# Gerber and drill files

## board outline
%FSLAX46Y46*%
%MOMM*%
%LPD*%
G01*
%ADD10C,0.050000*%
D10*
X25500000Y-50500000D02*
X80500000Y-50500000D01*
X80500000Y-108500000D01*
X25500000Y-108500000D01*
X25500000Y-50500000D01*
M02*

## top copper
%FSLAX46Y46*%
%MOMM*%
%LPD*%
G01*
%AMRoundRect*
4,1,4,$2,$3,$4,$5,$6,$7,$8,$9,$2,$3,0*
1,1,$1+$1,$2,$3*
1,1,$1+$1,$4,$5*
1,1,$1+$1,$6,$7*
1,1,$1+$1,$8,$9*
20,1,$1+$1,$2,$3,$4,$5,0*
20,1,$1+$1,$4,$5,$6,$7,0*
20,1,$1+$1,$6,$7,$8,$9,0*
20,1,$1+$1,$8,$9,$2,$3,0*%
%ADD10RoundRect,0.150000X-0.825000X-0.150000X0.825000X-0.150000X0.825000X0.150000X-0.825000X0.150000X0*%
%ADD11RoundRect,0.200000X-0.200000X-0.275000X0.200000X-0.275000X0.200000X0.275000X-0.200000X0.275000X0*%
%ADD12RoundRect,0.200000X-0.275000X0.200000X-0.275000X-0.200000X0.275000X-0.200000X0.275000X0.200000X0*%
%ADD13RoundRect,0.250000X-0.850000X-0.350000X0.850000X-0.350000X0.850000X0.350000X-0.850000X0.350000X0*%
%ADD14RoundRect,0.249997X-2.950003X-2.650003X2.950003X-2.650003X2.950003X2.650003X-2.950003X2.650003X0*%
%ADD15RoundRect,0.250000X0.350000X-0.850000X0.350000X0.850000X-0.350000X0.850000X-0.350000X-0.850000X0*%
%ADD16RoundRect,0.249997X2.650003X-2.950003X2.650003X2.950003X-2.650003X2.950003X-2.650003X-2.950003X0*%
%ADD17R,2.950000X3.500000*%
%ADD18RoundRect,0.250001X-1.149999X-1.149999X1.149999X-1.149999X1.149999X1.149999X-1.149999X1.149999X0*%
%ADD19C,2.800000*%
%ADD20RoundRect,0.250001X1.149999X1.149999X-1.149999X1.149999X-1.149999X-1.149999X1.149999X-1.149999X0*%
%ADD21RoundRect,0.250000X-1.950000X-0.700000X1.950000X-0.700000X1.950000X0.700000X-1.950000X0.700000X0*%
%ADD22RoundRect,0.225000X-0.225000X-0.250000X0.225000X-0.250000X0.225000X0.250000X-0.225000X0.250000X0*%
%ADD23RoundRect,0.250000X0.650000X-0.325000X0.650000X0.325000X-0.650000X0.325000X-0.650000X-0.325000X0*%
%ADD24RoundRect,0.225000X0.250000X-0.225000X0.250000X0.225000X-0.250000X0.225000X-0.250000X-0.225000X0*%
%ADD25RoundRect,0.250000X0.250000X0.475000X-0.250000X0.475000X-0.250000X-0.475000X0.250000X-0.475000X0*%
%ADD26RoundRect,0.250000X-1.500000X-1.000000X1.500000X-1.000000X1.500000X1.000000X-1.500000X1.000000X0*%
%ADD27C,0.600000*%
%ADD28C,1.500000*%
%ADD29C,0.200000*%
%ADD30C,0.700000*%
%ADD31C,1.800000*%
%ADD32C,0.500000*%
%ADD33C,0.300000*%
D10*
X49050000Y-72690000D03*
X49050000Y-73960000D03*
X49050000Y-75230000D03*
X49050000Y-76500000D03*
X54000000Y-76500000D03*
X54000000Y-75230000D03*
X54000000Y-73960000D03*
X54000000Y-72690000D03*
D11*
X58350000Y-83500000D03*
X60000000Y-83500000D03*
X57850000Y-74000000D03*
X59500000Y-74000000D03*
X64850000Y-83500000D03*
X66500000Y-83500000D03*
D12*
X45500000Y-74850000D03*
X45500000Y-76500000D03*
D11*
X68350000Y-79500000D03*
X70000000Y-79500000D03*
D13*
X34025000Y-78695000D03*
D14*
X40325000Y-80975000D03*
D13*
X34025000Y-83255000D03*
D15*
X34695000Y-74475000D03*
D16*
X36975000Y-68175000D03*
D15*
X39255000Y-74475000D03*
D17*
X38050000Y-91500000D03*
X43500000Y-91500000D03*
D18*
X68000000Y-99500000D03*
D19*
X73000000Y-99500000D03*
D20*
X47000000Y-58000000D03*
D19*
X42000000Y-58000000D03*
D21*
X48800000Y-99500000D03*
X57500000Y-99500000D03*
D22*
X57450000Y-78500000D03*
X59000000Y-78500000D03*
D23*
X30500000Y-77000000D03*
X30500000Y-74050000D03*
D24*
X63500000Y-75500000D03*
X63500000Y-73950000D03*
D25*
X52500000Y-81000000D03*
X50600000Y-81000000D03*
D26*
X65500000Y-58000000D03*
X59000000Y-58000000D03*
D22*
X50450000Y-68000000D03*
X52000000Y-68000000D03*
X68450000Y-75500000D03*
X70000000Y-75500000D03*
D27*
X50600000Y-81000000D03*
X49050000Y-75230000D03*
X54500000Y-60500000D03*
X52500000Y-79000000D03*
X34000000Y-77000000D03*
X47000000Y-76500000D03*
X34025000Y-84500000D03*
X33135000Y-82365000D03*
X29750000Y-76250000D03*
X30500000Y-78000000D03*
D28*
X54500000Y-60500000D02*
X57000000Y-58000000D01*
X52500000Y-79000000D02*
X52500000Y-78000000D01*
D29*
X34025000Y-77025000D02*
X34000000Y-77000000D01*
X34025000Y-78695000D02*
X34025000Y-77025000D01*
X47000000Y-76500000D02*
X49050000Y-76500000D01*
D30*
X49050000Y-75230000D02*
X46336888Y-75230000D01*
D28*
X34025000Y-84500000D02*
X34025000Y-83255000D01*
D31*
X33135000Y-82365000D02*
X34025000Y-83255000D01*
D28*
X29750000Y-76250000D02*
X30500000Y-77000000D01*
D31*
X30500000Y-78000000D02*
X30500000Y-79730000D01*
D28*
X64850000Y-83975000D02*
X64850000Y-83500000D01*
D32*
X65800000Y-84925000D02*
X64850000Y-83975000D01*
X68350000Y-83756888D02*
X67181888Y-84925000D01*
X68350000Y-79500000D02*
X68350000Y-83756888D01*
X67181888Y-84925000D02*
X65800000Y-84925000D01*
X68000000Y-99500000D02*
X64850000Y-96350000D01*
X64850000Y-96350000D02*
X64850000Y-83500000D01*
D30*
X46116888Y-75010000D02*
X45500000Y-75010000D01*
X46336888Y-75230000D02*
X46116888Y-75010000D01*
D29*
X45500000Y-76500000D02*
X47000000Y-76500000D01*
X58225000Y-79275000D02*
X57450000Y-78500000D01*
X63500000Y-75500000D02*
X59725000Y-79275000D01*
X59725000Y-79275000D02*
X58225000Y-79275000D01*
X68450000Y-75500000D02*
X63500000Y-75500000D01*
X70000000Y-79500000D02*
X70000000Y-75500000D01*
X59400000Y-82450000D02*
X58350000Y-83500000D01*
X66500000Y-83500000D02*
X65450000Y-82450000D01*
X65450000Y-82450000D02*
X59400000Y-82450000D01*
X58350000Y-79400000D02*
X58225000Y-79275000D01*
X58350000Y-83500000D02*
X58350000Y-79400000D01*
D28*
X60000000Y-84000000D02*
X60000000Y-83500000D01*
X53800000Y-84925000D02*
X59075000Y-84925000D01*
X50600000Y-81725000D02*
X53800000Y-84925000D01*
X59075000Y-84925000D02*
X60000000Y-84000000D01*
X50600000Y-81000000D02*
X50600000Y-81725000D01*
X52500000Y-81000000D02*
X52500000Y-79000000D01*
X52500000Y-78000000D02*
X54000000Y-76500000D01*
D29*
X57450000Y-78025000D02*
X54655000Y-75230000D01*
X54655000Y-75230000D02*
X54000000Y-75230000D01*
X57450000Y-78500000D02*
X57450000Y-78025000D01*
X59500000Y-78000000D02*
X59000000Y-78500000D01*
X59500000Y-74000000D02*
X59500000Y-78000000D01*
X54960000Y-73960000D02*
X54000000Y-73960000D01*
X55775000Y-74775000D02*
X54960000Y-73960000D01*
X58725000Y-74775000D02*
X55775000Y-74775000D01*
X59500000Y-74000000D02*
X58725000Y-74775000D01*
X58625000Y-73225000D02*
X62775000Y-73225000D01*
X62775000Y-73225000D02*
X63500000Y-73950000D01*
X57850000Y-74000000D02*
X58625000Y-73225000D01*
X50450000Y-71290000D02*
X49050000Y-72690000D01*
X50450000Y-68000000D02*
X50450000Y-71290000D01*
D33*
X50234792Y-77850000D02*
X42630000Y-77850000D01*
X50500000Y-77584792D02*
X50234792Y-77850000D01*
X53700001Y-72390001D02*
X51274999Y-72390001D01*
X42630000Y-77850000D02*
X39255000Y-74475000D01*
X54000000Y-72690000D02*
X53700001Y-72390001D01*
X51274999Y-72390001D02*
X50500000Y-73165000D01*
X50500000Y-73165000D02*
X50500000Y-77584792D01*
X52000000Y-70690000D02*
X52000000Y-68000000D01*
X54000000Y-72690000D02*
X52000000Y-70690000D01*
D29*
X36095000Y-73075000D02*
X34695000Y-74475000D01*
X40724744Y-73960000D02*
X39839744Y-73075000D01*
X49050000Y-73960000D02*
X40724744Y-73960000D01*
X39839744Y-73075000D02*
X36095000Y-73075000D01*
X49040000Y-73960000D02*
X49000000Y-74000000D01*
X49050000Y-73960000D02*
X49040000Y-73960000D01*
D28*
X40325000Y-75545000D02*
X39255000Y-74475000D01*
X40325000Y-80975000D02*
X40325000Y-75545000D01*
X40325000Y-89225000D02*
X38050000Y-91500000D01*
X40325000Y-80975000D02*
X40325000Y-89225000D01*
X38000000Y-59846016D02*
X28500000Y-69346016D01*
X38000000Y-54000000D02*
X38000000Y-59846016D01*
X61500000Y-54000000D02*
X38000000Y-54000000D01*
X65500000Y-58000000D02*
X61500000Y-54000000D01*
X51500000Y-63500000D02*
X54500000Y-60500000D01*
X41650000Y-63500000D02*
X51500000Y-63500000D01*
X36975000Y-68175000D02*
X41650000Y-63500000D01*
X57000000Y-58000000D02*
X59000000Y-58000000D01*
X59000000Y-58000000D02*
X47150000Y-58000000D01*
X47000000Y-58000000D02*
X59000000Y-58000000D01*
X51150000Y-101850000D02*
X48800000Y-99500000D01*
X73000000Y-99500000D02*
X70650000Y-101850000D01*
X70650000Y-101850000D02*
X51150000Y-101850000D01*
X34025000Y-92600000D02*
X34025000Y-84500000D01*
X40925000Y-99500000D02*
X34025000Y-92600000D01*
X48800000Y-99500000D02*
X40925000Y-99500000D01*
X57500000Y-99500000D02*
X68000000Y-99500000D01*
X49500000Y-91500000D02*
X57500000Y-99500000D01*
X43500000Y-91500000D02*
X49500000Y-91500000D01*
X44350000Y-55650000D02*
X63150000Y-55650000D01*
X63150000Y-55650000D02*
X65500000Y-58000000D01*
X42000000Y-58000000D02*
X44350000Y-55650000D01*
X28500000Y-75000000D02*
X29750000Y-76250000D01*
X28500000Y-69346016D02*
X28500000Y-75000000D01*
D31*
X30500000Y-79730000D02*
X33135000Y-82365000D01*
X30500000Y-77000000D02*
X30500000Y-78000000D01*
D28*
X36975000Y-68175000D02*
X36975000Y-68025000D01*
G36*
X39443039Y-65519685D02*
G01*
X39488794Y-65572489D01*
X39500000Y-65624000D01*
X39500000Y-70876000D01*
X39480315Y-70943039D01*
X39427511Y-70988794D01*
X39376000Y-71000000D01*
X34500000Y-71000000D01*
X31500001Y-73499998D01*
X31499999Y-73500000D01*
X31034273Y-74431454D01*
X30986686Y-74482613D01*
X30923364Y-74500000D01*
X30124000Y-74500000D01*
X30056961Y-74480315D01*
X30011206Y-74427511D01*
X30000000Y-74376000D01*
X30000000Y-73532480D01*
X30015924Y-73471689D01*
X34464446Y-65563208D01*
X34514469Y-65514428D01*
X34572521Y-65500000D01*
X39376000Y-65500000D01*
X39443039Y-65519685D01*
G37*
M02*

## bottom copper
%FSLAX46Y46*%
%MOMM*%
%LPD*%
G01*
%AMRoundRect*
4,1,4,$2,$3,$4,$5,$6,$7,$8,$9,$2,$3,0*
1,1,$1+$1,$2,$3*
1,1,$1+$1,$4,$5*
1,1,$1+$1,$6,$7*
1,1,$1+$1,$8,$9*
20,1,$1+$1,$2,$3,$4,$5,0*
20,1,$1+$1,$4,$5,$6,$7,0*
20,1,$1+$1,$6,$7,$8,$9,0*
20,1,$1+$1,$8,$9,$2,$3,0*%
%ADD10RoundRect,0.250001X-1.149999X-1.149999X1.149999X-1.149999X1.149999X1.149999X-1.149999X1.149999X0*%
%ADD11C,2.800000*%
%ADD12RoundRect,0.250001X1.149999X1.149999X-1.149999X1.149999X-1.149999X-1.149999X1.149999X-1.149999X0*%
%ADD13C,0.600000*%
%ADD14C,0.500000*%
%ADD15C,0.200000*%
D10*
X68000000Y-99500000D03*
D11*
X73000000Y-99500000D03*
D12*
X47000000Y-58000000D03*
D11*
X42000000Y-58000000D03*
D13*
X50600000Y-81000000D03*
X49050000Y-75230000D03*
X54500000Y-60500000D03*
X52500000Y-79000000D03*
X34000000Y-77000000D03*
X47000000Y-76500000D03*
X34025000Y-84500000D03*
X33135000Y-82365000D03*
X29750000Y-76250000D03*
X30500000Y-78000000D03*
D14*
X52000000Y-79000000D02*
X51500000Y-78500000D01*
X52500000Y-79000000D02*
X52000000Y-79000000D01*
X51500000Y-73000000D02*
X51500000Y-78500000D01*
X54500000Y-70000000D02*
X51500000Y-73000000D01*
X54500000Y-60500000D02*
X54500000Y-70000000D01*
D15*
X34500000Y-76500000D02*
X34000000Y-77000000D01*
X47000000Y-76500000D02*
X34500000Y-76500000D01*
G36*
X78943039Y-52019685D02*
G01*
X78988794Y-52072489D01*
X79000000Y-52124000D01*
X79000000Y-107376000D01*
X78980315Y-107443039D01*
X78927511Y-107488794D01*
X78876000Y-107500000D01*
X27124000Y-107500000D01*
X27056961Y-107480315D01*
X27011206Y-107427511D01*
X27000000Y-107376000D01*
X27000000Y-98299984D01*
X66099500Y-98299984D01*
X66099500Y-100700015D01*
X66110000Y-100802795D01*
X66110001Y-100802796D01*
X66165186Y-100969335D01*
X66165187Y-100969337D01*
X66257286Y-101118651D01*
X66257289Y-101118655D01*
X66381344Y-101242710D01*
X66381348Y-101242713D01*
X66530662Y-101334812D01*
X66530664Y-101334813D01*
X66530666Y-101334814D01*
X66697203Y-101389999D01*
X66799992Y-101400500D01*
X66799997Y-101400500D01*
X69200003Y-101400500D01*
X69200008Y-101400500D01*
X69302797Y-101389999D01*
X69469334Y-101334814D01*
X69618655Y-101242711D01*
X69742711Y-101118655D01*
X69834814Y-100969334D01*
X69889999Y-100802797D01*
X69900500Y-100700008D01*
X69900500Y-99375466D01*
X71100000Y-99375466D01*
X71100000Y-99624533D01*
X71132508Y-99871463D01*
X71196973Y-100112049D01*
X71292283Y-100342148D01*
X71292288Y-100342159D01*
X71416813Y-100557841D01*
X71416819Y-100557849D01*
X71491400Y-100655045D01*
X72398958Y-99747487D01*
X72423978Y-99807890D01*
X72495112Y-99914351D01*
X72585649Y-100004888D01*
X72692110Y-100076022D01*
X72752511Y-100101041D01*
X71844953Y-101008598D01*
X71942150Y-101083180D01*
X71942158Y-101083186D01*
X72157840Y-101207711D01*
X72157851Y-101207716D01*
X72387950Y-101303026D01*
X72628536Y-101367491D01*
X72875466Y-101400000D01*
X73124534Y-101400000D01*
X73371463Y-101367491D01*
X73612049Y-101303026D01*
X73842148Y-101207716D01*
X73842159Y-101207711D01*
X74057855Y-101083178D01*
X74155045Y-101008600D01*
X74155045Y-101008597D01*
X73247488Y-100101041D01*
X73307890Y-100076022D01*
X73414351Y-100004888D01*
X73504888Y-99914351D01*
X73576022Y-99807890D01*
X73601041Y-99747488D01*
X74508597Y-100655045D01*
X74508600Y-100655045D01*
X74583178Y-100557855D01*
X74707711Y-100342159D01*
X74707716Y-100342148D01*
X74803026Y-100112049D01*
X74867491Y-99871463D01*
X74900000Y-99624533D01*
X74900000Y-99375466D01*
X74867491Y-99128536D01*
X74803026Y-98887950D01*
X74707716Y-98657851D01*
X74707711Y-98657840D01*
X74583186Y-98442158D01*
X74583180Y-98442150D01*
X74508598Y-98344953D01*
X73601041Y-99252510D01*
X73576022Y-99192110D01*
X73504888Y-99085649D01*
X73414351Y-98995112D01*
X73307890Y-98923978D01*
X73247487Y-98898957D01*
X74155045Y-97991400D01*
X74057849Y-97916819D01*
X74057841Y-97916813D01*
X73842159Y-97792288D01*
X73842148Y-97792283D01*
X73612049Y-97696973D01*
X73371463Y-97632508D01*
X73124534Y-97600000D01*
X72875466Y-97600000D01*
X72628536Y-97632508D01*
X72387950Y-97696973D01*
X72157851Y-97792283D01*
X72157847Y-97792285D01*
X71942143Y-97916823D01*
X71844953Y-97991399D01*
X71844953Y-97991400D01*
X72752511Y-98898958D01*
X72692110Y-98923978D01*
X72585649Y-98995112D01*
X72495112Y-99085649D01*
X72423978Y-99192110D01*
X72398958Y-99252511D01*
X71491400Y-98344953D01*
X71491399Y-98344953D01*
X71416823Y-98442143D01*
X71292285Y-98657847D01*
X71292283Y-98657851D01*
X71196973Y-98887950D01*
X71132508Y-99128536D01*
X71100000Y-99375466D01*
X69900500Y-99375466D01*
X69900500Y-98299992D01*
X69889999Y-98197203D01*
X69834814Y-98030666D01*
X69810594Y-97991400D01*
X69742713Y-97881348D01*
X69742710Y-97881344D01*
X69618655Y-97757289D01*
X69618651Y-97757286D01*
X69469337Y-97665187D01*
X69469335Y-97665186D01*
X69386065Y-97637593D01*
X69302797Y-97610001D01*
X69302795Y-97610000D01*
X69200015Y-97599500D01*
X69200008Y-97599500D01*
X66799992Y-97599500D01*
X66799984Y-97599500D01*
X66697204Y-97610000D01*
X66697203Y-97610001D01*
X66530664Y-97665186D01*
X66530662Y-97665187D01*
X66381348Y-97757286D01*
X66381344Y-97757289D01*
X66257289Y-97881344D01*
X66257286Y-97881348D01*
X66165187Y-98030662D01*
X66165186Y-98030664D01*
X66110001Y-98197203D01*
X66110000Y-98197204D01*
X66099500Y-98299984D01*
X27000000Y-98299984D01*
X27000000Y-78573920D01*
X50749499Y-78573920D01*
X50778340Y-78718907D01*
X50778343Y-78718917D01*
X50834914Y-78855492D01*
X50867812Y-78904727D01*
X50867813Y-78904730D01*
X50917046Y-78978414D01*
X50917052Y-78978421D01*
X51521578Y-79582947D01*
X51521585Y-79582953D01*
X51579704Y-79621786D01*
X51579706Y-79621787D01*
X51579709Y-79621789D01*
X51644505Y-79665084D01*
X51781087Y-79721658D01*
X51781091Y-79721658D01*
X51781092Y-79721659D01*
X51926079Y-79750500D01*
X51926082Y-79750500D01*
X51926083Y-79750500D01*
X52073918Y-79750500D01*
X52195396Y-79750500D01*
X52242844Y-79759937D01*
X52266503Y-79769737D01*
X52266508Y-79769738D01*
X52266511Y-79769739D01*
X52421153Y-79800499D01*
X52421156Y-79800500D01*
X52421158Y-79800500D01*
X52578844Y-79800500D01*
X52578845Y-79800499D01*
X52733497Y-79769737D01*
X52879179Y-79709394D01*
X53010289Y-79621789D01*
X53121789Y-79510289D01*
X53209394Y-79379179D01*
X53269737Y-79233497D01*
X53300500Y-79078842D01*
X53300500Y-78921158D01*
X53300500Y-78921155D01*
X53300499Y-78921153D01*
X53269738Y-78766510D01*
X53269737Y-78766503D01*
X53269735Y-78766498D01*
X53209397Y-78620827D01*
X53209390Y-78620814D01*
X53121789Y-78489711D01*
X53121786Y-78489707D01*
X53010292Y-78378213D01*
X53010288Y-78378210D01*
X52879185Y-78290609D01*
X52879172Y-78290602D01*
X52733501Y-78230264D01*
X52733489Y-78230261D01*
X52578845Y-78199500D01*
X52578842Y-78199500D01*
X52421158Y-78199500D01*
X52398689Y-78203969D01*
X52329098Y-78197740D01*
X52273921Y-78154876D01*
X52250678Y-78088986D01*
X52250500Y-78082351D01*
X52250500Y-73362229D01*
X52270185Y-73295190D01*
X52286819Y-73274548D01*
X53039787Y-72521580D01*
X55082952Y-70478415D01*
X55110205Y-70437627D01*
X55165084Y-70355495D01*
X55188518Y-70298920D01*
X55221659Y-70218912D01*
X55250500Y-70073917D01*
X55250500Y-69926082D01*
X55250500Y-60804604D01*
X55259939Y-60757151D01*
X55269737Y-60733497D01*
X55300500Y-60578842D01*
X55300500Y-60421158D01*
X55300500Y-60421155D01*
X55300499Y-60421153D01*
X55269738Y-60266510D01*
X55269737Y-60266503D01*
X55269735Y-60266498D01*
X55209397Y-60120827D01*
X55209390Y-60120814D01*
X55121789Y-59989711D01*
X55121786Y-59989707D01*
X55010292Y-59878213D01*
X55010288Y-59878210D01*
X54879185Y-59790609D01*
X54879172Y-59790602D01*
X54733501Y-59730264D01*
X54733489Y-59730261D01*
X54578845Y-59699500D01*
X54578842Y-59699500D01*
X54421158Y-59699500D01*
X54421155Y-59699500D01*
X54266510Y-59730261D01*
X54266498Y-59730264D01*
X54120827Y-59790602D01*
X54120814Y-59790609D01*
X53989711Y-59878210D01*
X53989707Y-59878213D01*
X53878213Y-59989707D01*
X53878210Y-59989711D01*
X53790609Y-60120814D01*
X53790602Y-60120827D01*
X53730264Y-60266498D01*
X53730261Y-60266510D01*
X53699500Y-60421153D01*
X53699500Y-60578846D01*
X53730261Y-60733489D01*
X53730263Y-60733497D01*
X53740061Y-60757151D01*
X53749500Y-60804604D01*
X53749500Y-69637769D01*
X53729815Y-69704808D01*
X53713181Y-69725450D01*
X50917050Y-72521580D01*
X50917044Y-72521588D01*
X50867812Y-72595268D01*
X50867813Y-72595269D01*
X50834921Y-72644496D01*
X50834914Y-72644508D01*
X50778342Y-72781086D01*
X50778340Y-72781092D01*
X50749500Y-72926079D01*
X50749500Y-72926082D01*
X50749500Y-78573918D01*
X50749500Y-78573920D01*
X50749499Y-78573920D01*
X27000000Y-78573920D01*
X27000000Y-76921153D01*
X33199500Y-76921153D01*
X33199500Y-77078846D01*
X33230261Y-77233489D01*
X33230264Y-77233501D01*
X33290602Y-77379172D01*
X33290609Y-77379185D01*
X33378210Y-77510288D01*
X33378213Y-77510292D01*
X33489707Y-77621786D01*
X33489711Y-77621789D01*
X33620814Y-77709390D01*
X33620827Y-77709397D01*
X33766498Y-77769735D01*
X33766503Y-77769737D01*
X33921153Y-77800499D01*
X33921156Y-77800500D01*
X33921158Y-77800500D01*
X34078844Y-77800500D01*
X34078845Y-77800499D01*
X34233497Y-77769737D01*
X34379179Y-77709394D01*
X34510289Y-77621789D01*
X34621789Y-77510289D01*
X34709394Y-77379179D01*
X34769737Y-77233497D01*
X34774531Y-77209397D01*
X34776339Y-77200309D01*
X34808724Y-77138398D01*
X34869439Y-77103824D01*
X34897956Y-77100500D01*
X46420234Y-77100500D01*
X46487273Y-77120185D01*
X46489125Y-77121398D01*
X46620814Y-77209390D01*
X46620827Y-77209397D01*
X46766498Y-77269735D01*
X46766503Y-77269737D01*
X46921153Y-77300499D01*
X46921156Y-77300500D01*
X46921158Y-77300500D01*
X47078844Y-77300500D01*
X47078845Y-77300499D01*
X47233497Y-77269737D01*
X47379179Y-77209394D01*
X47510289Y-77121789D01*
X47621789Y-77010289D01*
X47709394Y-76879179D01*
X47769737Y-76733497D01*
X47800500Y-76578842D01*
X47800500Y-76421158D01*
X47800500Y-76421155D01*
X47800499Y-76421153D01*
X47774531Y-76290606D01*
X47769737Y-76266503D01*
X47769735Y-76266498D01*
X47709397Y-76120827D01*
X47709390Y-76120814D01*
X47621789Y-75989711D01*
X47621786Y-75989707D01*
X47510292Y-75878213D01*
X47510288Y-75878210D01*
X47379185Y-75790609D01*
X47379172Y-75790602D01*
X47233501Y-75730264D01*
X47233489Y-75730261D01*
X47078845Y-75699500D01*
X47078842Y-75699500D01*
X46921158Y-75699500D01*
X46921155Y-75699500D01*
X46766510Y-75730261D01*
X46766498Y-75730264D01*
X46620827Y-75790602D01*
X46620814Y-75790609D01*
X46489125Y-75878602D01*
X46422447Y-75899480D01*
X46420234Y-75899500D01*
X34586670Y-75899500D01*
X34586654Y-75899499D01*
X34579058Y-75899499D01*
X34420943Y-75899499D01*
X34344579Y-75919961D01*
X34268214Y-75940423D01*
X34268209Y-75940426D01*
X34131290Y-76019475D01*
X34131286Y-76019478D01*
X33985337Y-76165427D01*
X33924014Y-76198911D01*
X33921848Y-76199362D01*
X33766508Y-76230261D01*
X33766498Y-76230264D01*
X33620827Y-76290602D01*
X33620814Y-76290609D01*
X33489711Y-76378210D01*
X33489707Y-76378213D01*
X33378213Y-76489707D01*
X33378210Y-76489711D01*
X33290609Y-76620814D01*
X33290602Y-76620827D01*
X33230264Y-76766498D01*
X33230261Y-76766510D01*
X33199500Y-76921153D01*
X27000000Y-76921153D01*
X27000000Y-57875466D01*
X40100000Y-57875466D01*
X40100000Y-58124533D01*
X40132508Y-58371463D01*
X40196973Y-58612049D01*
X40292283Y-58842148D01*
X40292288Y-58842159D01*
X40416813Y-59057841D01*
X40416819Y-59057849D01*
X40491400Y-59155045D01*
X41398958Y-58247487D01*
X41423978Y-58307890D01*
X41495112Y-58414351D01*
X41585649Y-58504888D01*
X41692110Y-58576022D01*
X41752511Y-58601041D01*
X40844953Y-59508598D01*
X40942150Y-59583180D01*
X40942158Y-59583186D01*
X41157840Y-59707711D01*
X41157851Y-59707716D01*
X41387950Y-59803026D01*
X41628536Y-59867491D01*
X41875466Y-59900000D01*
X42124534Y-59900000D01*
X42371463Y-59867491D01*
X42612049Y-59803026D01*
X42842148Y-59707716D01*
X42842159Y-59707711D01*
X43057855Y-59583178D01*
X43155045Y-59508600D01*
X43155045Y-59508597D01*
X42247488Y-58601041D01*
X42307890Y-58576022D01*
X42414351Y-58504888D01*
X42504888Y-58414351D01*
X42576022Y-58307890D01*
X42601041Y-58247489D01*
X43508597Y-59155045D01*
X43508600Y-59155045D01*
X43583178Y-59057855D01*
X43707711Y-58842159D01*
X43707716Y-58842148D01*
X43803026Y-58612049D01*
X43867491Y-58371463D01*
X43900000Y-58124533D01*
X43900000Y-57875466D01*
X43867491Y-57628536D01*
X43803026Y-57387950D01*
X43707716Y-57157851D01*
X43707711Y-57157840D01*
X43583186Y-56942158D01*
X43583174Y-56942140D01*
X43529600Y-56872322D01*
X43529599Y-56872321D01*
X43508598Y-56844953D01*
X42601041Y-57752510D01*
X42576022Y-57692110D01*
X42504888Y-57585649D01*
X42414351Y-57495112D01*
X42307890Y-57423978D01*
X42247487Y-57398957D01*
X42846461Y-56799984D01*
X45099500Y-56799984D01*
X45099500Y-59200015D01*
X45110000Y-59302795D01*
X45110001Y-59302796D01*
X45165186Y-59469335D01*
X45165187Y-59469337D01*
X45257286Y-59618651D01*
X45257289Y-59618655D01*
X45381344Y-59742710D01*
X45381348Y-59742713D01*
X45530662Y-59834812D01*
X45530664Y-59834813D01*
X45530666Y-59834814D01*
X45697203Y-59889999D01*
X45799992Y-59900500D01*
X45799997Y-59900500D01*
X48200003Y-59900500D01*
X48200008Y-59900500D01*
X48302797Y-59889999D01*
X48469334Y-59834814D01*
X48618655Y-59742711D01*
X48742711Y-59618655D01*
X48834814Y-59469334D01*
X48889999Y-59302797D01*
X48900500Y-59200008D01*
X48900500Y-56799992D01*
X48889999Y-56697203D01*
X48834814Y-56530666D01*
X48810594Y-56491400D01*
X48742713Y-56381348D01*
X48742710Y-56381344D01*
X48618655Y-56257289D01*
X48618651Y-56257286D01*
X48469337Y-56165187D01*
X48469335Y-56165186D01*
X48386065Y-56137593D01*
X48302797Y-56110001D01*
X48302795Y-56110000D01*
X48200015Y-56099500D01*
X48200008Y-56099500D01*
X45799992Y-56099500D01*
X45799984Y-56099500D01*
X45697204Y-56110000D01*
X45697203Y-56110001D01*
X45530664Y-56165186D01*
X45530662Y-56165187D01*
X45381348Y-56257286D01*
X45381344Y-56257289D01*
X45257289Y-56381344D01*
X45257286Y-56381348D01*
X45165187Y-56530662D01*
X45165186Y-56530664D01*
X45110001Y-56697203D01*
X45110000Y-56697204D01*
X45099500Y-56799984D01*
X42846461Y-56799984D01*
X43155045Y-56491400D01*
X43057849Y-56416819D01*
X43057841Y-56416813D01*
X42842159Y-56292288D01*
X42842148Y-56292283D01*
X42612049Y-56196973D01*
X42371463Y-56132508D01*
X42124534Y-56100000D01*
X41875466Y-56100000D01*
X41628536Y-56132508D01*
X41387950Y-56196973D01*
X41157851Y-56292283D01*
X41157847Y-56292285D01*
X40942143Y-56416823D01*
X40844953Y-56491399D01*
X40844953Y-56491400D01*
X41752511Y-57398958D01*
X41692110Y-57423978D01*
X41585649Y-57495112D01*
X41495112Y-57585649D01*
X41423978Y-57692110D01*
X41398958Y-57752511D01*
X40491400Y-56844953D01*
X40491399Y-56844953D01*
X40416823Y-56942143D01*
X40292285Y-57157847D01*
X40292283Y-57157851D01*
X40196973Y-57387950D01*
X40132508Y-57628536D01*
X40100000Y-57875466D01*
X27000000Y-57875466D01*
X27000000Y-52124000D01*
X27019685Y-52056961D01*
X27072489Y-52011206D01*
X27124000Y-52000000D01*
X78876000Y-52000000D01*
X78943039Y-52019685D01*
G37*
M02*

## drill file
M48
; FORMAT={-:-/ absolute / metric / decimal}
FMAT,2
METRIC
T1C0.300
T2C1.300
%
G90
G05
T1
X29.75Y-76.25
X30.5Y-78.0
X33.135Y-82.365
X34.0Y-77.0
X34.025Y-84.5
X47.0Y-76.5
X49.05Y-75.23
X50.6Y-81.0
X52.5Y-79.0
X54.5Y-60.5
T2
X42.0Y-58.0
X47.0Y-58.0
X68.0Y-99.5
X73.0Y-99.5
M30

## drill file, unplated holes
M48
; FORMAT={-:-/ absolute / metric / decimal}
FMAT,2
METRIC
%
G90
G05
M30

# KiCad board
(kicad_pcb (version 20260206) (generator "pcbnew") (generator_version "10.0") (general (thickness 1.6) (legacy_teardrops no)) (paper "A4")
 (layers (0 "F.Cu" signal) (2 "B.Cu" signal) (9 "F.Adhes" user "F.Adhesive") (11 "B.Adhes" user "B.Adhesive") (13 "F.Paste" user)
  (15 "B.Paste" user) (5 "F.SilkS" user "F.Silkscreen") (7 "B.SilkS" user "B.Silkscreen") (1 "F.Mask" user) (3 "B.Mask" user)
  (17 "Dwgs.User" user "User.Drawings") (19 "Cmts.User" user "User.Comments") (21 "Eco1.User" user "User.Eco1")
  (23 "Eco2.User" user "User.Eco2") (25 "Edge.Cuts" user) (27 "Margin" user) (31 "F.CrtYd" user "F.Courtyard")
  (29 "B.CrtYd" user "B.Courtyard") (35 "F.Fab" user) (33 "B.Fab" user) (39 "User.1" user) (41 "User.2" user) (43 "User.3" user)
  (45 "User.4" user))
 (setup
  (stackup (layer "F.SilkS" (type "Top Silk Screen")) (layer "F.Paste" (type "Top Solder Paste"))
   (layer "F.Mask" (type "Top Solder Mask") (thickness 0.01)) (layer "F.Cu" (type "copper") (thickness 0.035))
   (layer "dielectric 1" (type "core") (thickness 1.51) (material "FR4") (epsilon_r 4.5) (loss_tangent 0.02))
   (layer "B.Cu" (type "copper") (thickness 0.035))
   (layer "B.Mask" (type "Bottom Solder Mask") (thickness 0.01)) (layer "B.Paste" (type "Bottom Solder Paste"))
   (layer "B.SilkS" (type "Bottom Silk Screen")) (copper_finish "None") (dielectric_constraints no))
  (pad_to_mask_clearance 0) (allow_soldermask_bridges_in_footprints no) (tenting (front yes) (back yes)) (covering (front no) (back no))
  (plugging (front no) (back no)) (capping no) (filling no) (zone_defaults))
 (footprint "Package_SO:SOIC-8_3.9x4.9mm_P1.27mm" (layer "F.Cu") (at 51.525 74.595)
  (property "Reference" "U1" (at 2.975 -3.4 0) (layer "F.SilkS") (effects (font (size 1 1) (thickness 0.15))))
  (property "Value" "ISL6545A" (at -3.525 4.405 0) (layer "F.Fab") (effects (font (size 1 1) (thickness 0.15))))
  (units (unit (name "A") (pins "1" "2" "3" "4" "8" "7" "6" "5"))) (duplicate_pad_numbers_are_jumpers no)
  (pad "1" smd roundrect (at -2.475 -1.905) (size 1.95 0.6) (layers "F.Cu" "F.Mask" "F.Paste") (roundrect_rratio 0.25) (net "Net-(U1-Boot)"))
  (pad "2" smd roundrect (at -2.475 -0.635) (size 1.95 0.6) (layers "F.Cu" "F.Mask" "F.Paste") (roundrect_rratio 0.25) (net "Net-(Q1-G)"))
  (pad "3" smd roundrect (at -2.475 0.635) (size 1.95 0.6) (layers "F.Cu" "F.Mask" "F.Paste") (roundrect_rratio 0.25) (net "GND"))
  (pad "4" smd roundrect (at -2.475 1.905) (size 1.95 0.6) (layers "F.Cu" "F.Mask" "F.Paste") (roundrect_rratio 0.25) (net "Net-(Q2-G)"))
  (pad "5" smd roundrect (at 2.475 1.905) (size 1.95 0.6) (layers "F.Cu" "F.Mask" "F.Paste") (roundrect_rratio 0.25) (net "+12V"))
  (pad "6" smd roundrect (at 2.475 0.635) (size 1.95 0.6) (layers "F.Cu" "F.Mask" "F.Paste") (roundrect_rratio 0.25) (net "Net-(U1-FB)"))
  (pad "7" smd roundrect (at 2.475 -0.635) (size 1.95 0.6) (layers "F.Cu" "F.Mask" "F.Paste") (roundrect_rratio 0.25)
   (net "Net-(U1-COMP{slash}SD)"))
  (pad "8" smd roundrect (at 2.475 -1.905) (size 1.95 0.6) (layers "F.Cu" "F.Mask" "F.Paste") (roundrect_rratio 0.25) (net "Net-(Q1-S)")))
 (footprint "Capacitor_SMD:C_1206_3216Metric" (layer "F.Cu") (at 30.5 75.525 90)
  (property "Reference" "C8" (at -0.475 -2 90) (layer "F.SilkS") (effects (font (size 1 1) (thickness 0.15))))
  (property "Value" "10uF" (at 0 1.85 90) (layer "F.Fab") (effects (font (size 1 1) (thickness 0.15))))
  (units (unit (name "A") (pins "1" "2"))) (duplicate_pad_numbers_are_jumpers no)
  (pad "1" smd roundrect (at -1.475 0 90) (size 1.15 1.8) (layers "F.Cu" "F.Mask" "F.Paste") (roundrect_rratio 0.217391) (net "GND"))
  (pad "2" smd roundrect (at 1.475 0 90) (size 1.15 1.8) (layers "F.Cu" "F.Mask" "F.Paste") (roundrect_rratio 0.217391) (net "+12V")))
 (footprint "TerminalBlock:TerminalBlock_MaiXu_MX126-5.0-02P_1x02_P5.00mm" (layer "F.Cu") (at 47 58 180)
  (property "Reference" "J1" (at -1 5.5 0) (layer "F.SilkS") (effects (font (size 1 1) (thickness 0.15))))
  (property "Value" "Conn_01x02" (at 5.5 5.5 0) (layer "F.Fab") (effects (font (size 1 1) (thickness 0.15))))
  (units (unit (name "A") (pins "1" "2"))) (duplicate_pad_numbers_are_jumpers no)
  (pad "1" thru_hole roundrect (at 0 0 180) (size 2.8 2.8) (drill 1.3) (layers "*.Cu" "*.Mask") (remove_unused_layers no)
   (roundrect_rratio 0.089286) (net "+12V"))
  (pad "2" thru_hole circle (at 5 0 180) (size 2.8 2.8) (drill 1.3) (layers "*.Cu" "*.Mask") (remove_unused_layers no) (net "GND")))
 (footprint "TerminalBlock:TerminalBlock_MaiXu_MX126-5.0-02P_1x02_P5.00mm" (layer "F.Cu") (at 68 99.5)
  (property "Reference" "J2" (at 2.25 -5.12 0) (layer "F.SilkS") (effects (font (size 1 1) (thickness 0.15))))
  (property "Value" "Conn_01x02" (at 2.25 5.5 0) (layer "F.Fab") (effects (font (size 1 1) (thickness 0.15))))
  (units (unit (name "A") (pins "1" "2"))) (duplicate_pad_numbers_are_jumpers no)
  (pad "1" thru_hole roundrect (at 0 0) (size 2.8 2.8) (drill 1.3) (layers "*.Cu" "*.Mask") (remove_unused_layers no)
   (roundrect_rratio 0.089286) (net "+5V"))
  (pad "2" thru_hole circle (at 5 0) (size 2.8 2.8) (drill 1.3) (layers "*.Cu" "*.Mask") (remove_unused_layers no) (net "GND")))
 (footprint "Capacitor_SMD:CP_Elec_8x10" (layer "F.Cu") (at 62.25 58)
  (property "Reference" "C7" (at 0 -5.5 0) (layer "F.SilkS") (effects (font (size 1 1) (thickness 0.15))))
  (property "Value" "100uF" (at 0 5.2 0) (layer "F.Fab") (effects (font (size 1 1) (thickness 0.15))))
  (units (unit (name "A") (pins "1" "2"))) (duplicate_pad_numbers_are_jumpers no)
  (pad "1" smd roundrect (at -3.25 0) (size 3.5 2.5) (layers "F.Cu" "F.Mask" "F.Paste") (roundrect_rratio 0.1) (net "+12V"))
  (pad "2" smd roundrect (at 3.25 0) (size 3.5 2.5) (layers "F.Cu" "F.Mask" "F.Paste") (roundrect_rratio 0.1) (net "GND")))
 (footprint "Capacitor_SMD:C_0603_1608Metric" (layer "F.Cu") (at 63.5 74.725 90)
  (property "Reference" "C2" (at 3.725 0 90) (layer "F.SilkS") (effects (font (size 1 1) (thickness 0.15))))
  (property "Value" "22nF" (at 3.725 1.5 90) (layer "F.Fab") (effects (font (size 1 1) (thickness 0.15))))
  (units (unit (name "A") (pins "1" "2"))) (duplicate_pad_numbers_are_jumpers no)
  (pad "1" smd roundrect (at -0.775 0 90) (size 0.9 0.95) (layers "F.Cu" "F.Mask" "F.Paste") (roundrect_rratio 0.25) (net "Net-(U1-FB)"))
  (pad "2" smd roundrect (at 0.775 0 90) (size 0.9 0.95) (layers "F.Cu" "F.Mask" "F.Paste") (roundrect_rratio 0.25) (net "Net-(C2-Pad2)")))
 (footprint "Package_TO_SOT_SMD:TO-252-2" (layer "F.Cu") (at 39.065 80.975)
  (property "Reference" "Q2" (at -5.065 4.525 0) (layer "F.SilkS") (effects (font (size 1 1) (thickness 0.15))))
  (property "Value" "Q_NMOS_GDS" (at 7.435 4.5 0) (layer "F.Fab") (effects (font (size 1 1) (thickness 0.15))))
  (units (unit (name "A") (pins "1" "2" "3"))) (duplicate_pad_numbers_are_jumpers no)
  (pad "" smd roundrect (at -0.415 -1.525) (size 3.05 2.75) (layers "F.Paste") (roundrect_rratio 0.090909))
  (pad "" smd roundrect (at -0.415 1.525) (size 3.05 2.75) (layers "F.Paste") (roundrect_rratio 0.090909))
  (pad "" smd roundrect (at 2.935 -1.525) (size 3.05 2.75) (layers "F.Paste") (roundrect_rratio 0.090909))
  (pad "" smd roundrect (at 2.935 1.525) (size 3.05 2.75) (layers "F.Paste") (roundrect_rratio 0.090909))
  (pad "1" smd roundrect (at -5.04 -2.28) (size 2.2 1.2) (layers "F.Cu" "F.Mask" "F.Paste") (roundrect_rratio 0.208333) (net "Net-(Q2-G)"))
  (pad "2" smd roundrect (at 1.26 0) (size 6.4 5.8) (layers "F.Cu" "F.Mask") (roundrect_rratio 0.043103) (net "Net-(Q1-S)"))
  (pad "3" smd roundrect (at -5.04 2.28) (size 2.2 1.2) (layers "F.Cu" "F.Mask" "F.Paste") (roundrect_rratio 0.208333) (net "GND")))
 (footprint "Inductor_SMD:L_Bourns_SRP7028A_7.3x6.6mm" (layer "F.Cu") (at 40.775 91.5)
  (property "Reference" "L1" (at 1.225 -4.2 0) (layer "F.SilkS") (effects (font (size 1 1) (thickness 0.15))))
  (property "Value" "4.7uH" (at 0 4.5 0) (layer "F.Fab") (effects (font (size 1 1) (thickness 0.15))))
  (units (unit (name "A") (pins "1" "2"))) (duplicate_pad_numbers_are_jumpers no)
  (pad "1" smd rect (at -2.725 0) (size 2.95 3.5) (layers "F.Cu" "F.Mask" "F.Paste") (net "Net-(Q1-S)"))
  (pad "2" smd rect (at 2.725 0) (size 2.95 3.5) (layers "F.Cu" "F.Mask" "F.Paste") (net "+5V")))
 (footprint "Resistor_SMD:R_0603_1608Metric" (layer "F.Cu") (at 45.5 75.675 -90)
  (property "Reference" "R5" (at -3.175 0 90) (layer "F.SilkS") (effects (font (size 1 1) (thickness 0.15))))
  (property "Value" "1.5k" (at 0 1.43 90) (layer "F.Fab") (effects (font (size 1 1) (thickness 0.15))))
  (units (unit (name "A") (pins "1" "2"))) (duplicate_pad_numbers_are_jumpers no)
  (pad "1" smd roundrect (at -0.825 0 270) (size 0.8 0.95) (layers "F.Cu" "F.Mask" "F.Paste") (roundrect_rratio 0.25) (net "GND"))
  (pad "2" smd roundrect (at 0.825 0 270) (size 0.8 0.95) (layers "F.Cu" "F.Mask" "F.Paste") (roundrect_rratio 0.25) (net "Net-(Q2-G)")))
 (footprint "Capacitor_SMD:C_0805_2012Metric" (layer "F.Cu") (at 51.55 81 180)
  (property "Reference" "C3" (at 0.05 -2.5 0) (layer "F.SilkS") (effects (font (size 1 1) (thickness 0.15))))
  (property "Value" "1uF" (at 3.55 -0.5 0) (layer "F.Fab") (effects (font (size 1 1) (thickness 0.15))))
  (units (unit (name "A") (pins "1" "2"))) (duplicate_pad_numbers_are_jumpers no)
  (pad "1" smd roundrect (at -0.95 0 180) (size 1 1.45) (layers "F.Cu" "F.Mask" "F.Paste") (roundrect_rratio 0.25) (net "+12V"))
  (pad "2" smd roundrect (at 0.95 0 180) (size 1 1.45) (layers "F.Cu" "F.Mask" "F.Paste") (roundrect_rratio 0.25) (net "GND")))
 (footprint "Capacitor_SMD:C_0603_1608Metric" (layer "F.Cu") (at 51.225 68)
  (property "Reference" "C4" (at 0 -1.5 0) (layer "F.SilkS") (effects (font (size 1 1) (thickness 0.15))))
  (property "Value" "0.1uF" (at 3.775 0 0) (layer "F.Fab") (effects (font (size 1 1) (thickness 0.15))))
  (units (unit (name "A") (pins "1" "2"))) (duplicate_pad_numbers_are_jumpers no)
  (pad "1" smd roundrect (at -0.775 0) (size 0.9 0.95) (layers "F.Cu" "F.Mask" "F.Paste") (roundrect_rratio 0.25) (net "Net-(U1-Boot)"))
  (pad "2" smd roundrect (at 0.775 0) (size 0.9 0.95) (layers "F.Cu" "F.Mask" "F.Paste") (roundrect_rratio 0.25) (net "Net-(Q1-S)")))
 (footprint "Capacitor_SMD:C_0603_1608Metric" (layer "F.Cu") (at 69.225 75.5)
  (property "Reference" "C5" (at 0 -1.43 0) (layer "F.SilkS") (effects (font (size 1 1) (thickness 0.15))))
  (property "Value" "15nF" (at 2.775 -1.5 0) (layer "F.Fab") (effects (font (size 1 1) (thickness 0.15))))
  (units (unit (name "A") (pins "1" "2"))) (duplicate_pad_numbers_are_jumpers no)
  (pad "1" smd roundrect (at -0.775 0) (size 0.9 0.95) (layers "F.Cu" "F.Mask" "F.Paste") (roundrect_rratio 0.25) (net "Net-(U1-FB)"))
  (pad "2" smd roundrect (at 0.775 0) (size 0.9 0.95) (layers "F.Cu" "F.Mask" "F.Paste") (roundrect_rratio 0.25) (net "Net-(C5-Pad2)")))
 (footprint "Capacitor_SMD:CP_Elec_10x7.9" (layer "F.Cu") (at 53.15 99.5)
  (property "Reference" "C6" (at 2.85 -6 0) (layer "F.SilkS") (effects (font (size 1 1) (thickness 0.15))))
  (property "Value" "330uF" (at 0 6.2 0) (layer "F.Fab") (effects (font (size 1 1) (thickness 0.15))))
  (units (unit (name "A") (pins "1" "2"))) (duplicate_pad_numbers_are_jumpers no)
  (pad "1" smd roundrect (at -4.35 0) (size 4.4 1.9) (layers "F.Cu" "F.Mask" "F.Paste") (roundrect_rratio 0.131579) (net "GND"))
  (pad "2" smd roundrect (at 4.35 0) (size 4.4 1.9) (layers "F.Cu" "F.Mask" "F.Paste") (roundrect_rratio 0.131579) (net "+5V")))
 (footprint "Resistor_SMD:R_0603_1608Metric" (layer "F.Cu") (at 65.675 83.5)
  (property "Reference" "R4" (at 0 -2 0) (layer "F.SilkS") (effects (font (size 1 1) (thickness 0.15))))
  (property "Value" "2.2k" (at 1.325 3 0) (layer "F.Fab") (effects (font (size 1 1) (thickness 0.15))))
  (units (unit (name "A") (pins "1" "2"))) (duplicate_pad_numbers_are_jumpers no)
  (pad "1" smd roundrect (at -0.825 0) (size 0.8 0.95) (layers "F.Cu" "F.Mask" "F.Paste") (roundrect_rratio 0.25) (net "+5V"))
  (pad "2" smd roundrect (at 0.825 0) (size 0.8 0.95) (layers "F.Cu" "F.Mask" "F.Paste") (roundrect_rratio 0.25) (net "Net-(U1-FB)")))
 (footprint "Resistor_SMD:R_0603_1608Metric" (layer "F.Cu") (at 59.175 83.5)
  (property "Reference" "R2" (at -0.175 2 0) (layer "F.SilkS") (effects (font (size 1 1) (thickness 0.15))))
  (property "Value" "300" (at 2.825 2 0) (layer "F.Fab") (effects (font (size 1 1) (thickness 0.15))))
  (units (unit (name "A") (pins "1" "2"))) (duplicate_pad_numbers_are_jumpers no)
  (pad "1" smd roundrect (at -0.825 0) (size 0.8 0.95) (layers "F.Cu" "F.Mask" "F.Paste") (roundrect_rratio 0.25) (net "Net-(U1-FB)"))
  (pad "2" smd roundrect (at 0.825 0) (size 0.8 0.95) (layers "F.Cu" "F.Mask" "F.Paste") (roundrect_rratio 0.25) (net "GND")))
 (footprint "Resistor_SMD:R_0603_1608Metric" (layer "F.Cu") (at 58.675 74)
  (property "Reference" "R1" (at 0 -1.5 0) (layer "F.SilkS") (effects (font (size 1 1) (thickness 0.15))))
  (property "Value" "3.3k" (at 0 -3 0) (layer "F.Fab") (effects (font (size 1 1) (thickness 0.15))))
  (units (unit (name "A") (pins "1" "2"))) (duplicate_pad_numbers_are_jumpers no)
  (pad "1" smd roundrect (at -0.825 0) (size 0.8 0.95) (layers "F.Cu" "F.Mask" "F.Paste") (roundrect_rratio 0.25) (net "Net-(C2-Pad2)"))
  (pad "2" smd roundrect (at 0.825 0) (size 0.8 0.95) (layers "F.Cu" "F.Mask" "F.Paste") (roundrect_rratio 0.25)
   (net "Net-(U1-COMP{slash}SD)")))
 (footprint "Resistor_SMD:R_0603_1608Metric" (layer "F.Cu") (at 69.175 79.5)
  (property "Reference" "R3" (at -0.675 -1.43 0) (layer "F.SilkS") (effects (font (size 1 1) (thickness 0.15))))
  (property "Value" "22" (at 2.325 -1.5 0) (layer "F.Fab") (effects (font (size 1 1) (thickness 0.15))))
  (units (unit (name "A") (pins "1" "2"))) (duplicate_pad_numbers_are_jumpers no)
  (pad "1" smd roundrect (at -0.825 0) (size 0.8 0.95) (layers "F.Cu" "F.Mask" "F.Paste") (roundrect_rratio 0.25) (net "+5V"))
  (pad "2" smd roundrect (at 0.825 0) (size 0.8 0.95) (layers "F.Cu" "F.Mask" "F.Paste") (roundrect_rratio 0.25) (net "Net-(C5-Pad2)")))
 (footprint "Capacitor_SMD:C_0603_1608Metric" (layer "F.Cu") (at 58.225 78.5)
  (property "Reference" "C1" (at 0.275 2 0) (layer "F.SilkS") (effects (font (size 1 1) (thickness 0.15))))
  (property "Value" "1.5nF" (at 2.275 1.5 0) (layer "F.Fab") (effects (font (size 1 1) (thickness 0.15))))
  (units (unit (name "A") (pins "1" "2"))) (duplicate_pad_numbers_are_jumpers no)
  (pad "1" smd roundrect (at -0.775 0) (size 0.9 0.95) (layers "F.Cu" "F.Mask" "F.Paste") (roundrect_rratio 0.25) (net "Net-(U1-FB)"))
  (pad "2" smd roundrect (at 0.775 0) (size 0.9 0.95) (layers "F.Cu" "F.Mask" "F.Paste") (roundrect_rratio 0.25)
   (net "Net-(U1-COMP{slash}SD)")))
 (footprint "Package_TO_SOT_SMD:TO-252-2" (layer "F.Cu") (at 36.975 69.435 90)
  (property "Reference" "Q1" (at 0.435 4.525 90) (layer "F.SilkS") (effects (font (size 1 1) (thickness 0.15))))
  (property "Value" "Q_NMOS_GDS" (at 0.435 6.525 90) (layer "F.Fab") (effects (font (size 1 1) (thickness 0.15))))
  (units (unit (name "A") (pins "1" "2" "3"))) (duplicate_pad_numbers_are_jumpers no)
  (pad "" smd roundrect (at -0.415 -1.525 90) (size 3.05 2.75) (layers "F.Paste") (roundrect_rratio 0.090909))
  (pad "" smd roundrect (at -0.415 1.525 90) (size 3.05 2.75) (layers "F.Paste") (roundrect_rratio 0.090909))
  (pad "" smd roundrect (at 2.935 -1.525 90) (size 3.05 2.75) (layers "F.Paste") (roundrect_rratio 0.090909))
  (pad "" smd roundrect (at 2.935 1.525 90) (size 3.05 2.75) (layers "F.Paste") (roundrect_rratio 0.090909))
  (pad "1" smd roundrect (at -5.04 -2.28 90) (size 2.2 1.2) (layers "F.Cu" "F.Mask" "F.Paste") (roundrect_rratio 0.208333)
   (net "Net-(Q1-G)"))
  (pad "2" smd roundrect (at 1.26 0 90) (size 6.4 5.8) (layers "F.Cu" "F.Mask") (roundrect_rratio 0.043103) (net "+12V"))
  (pad "3" smd roundrect (at -5.04 2.28 90) (size 2.2 1.2) (layers "F.Cu" "F.Mask" "F.Paste") (roundrect_rratio 0.208333) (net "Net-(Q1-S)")))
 (gr_rect (start 25.5 50.5) (end 80.5 108.5) (stroke (width 0.05) (type default)) (fill no) (layer "Edge.Cuts"))
 (segment (start 57.45 78.025) (end 54.655 75.23) (width 0.2) (layer "F.Cu") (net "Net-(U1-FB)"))
 (segment (start 59.725 79.275) (end 58.225 79.275) (width 0.2) (layer "F.Cu") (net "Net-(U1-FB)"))
 (segment (start 65.45 82.45) (end 59.4 82.45) (width 0.2) (layer "F.Cu") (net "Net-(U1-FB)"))
 (segment (start 59.4 82.45) (end 58.35 83.5) (width 0.2) (layer "F.Cu") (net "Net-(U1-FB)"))
 (segment (start 58.225 79.275) (end 57.45 78.5) (width 0.2) (layer "F.Cu") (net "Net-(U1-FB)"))
 (segment (start 63.5 75.5) (end 59.725 79.275) (width 0.2) (layer "F.Cu") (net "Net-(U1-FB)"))
 (segment (start 58.35 79.4) (end 58.225 79.275) (width 0.2) (layer "F.Cu") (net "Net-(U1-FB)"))
 (segment (start 66.5 83.5) (end 65.45 82.45) (width 0.2) (layer "F.Cu") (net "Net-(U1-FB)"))
 (segment (start 54.655 75.23) (end 54 75.23) (width 0.2) (layer "F.Cu") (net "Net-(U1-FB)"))
 (segment (start 57.45 78.5) (end 57.45 78.025) (width 0.2) (layer "F.Cu") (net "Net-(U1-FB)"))
 (segment (start 68.45 75.5) (end 63.5 75.5) (width 0.2) (layer "F.Cu") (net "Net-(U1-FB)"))
 (segment (start 58.35 83.5) (end 58.35 79.4) (width 0.2) (layer "F.Cu") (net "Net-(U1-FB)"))
 (segment (start 50.45 71.29) (end 49.05 72.69) (width 0.2) (layer "F.Cu") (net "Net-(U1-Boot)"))
 (segment (start 50.45 68) (end 50.45 71.29) (width 0.2) (layer "F.Cu") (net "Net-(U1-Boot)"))
 (segment (start 47 58) (end 59 58) (width 1.5) (layer "F.Cu") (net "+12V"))
 (segment (start 57 58) (end 59 58) (width 1.5) (layer "F.Cu") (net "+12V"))
 (segment (start 52.5 78) (end 54 76.5) (width 1.5) (layer "F.Cu") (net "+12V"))
 (segment (start 51.5 63.5) (end 54.5 60.5) (width 1.5) (layer "F.Cu") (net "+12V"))
 (segment (start 59 58) (end 47.15 58) (width 1.5) (layer "F.Cu") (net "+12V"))
 (segment (start 36.975 68.175) (end 36.975 68.025) (width 1.5) (layer "F.Cu") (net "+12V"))
 (segment (start 52.5 79) (end 52.5 78) (width 1.5) (layer "F.Cu") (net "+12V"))
 (segment (start 36.975 68.175) (end 41.65 63.5) (width 1.5) (layer "F.Cu") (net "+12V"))
 (segment (start 52.5 81) (end 52.5 79) (width 1.5) (layer "F.Cu") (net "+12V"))
 (segment (start 41.65 63.5) (end 51.5 63.5) (width 1.5) (layer "F.Cu") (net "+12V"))
 (segment (start 54.5 60.5) (end 57 58) (width 1.5) (layer "F.Cu") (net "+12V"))
 (via (at 52.5 79) (size 0.6) (drill 0.3) (layers "F.Cu" "B.Cu") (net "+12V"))
 (via (at 54.5 60.5) (size 0.6) (drill 0.3) (layers "F.Cu" "B.Cu") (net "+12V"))
 (segment (start 52.5 79) (end 52 79) (width 0.5) (layer "B.Cu") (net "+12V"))
 (segment (start 52 79) (end 51.5 78.5) (width 0.5) (layer "B.Cu") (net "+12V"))
 (segment (start 54.5 70) (end 51.5 73) (width 0.5) (layer "B.Cu") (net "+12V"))
 (segment (start 51.5 73) (end 51.5 78.5) (width 0.5) (layer "B.Cu") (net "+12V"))
 (segment (start 54.5 60.5) (end 54.5 70) (width 0.5) (layer "B.Cu") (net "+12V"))
 (segment (start 28.5 75) (end 29.75 76.25) (width 1.5) (layer "F.Cu") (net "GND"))
 (segment (start 30.5 79.73) (end 33.135 82.365) (width 1.8) (layer "F.Cu") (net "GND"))
 (segment (start 42 58) (end 44.35 55.65) (width 1.5) (layer "F.Cu") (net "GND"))
 (segment (start 53.8 84.925) (end 59.075 84.925) (width 1.5) (layer "F.Cu") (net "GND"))
 (segment (start 59.075 84.925) (end 60 84) (width 1.5) (layer "F.Cu") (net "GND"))
 (segment (start 44.35 55.65) (end 63.15 55.65) (width 1.5) (layer "F.Cu") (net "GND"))
 (segment (start 30.5 78) (end 30.5 79.73) (width 1.8) (layer "F.Cu") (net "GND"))
 (segment (start 46.336888 75.23) (end 46.116888 75.01) (width 0.7) (layer "F.Cu") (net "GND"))
 (segment (start 60 84) (end 60 83.5) (width 1.5) (layer "F.Cu") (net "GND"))
 (segment (start 63.15 55.65) (end 65.5 58) (width 1.5) (layer "F.Cu") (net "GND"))
 (segment (start 70.65 101.85) (end 51.15 101.85) (width 1.5) (layer "F.Cu") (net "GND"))
 (segment (start 51.15 101.85) (end 48.8 99.5) (width 1.5) (layer "F.Cu") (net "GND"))
 (segment (start 73 99.5) (end 70.65 101.85) (width 1.5) (layer "F.Cu") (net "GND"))
 (segment (start 61.5 54) (end 38 54) (width 1.5) (layer "F.Cu") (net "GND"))
 (segment (start 34.025 84.5) (end 34.025 83.255) (width 1.5) (layer "F.Cu") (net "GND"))
 (segment (start 29.75 76.25) (end 30.5 77) (width 1.5) (layer "F.Cu") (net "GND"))
 (segment (start 34.025 92.6) (end 34.025 84.5) (width 1.5) (layer "F.Cu") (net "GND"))
 (segment (start 50.6 81.725) (end 53.8 84.925) (width 1.5) (layer "F.Cu") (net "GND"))
 (segment (start 38 59.846016) (end 28.5 69.346016) (width 1.5) (layer "F.Cu") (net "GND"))
 (segment (start 46.116888 75.01) (end 45.5 75.01) (width 0.7) (layer "F.Cu") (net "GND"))
 (segment (start 33.135 82.365) (end 34.025 83.255) (width 1.8) (layer "F.Cu") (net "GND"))
 (segment (start 49.05 75.23) (end 46.336888 75.23) (width 0.7) (layer "F.Cu") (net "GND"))
 (segment (start 30.5 77) (end 30.5 78) (width 1.8) (layer "F.Cu") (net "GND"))
 (segment (start 40.925 99.5) (end 34.025 92.6) (width 1.5) (layer "F.Cu") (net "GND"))
 (segment (start 28.5 69.346016) (end 28.5 75) (width 1.5) (layer "F.Cu") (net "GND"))
 (segment (start 38 54) (end 38 59.846016) (width 1.5) (layer "F.Cu") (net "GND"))
 (segment (start 65.5 58) (end 61.5 54) (width 1.5) (layer "F.Cu") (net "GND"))
 (segment (start 50.6 81) (end 50.6 81.725) (width 1.5) (layer "F.Cu") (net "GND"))
 (segment (start 48.8 99.5) (end 40.925 99.5) (width 1.5) (layer "F.Cu") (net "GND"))
 (via (at 29.75 76.25) (size 0.6) (drill 0.3) (layers "F.Cu" "B.Cu") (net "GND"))
 (via (at 34.025 84.5) (size 0.6) (drill 0.3) (layers "F.Cu" "B.Cu") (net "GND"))
 (via (at 49.05 75.23) (size 0.6) (drill 0.3) (layers "F.Cu" "B.Cu") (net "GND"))
 (via (at 50.6 81) (size 0.6) (drill 0.3) (layers "F.Cu" "B.Cu") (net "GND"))
 (via (at 33.135 82.365) (size 0.6) (drill 0.3) (layers "F.Cu" "B.Cu") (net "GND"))
 (via (at 30.5 78) (size 0.6) (drill 0.3) (layers "F.Cu" "B.Cu") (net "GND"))
 (segment (start 58.725 74.775) (end 55.775 74.775) (width 0.2) (layer "F.Cu") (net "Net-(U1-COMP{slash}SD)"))
 (segment (start 59.5 78) (end 59 78.5) (width 0.2) (layer "F.Cu") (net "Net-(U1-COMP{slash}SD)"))
 (segment (start 55.775 74.775) (end 54.96 73.96) (width 0.2) (layer "F.Cu") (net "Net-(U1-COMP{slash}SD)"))
 (segment (start 59.5 74) (end 59.5 78) (width 0.2) (layer "F.Cu") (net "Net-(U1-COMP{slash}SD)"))
 (segment (start 54.96 73.96) (end 54 73.96) (width 0.2) (layer "F.Cu") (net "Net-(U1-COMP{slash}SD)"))
 (segment (start 59.5 74) (end 58.725 74.775) (width 0.2) (layer "F.Cu") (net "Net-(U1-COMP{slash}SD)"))
 (segment (start 67.181888 84.925) (end 65.8 84.925) (width 0.5) (layer "F.Cu") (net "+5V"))
 (segment (start 68 99.5) (end 64.85 96.35) (width 0.5) (layer "F.Cu") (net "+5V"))
 (segment (start 68.35 83.756888) (end 67.181888 84.925) (width 0.5) (layer "F.Cu") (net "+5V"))
 (segment (start 57.5 99.5) (end 68 99.5) (width 1.5) (layer "F.Cu") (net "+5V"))
 (segment (start 43.5 91.5) (end 49.5 91.5) (width 1.5) (layer "F.Cu") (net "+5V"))
 (segment (start 65.8 84.925) (end 64.85 83.975) (width 0.5) (layer "F.Cu") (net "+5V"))
 (segment (start 64.85 96.35) (end 64.85 83.5) (width 0.5) (layer "F.Cu") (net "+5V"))
 (segment (start 49.5 91.5) (end 57.5 99.5) (width 1.5) (layer "F.Cu") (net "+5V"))
 (segment (start 68.35 79.5) (end 68.35 83.756888) (width 0.5) (layer "F.Cu") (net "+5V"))
 (segment (start 64.85 83.975) (end 64.85 83.5) (width 1.5) (layer "F.Cu") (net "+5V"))
 (segment (start 58.625 73.225) (end 62.775 73.225) (width 0.2) (layer "F.Cu") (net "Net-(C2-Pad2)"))
 (segment (start 57.85 74) (end 58.625 73.225) (width 0.2) (layer "F.Cu") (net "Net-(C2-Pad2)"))
 (segment (start 62.775 73.225) (end 63.5 73.95) (width 0.2) (layer "F.Cu") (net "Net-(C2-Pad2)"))
 (segment (start 40.325 80.975) (end 40.325 75.545) (width 1.5) (layer "F.Cu") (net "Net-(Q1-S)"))
 (segment (start 54 72.69) (end 53.700001 72.390001) (width 0.3) (layer "F.Cu") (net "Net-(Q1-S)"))
 (segment (start 53.700001 72.390001) (end 51.274999 72.390001) (width 0.3) (layer "F.Cu") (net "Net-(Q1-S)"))
 (segment (start 54 72.69) (end 52 70.69) (width 0.3) (layer "F.Cu") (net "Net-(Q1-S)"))
 (segment (start 50.5 73.165) (end 50.5 77.584792) (width 0.3) (layer "F.Cu") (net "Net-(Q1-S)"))
 (segment (start 52 70.69) (end 52 68) (width 0.3) (layer "F.Cu") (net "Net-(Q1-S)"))
 (segment (start 50.5 77.584792) (end 50.234792 77.85) (width 0.3) (layer "F.Cu") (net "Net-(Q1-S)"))
 (segment (start 40.325 80.975) (end 40.325 89.225) (width 1.5) (layer "F.Cu") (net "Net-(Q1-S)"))
 (segment (start 51.274999 72.390001) (end 50.5 73.165) (width 0.3) (layer "F.Cu") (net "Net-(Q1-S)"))
 (segment (start 42.63 77.85) (end 39.255 74.475) (width 0.3) (layer "F.Cu") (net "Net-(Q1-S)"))
 (segment (start 40.325 89.225) (end 38.05 91.5) (width 1.5) (layer "F.Cu") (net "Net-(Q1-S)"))
 (segment (start 50.234792 77.85) (end 42.63 77.85) (width 0.3) (layer "F.Cu") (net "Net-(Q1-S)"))
 (segment (start 40.325 75.545) (end 39.255 74.475) (width 1.5) (layer "F.Cu") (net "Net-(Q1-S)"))
 (segment (start 70 79.5) (end 70 75.5) (width 0.2) (layer "F.Cu") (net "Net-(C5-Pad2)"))
 (segment (start 36.095 73.075) (end 34.695 74.475) (width 0.2) (layer "F.Cu") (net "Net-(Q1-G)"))
 (segment (start 49.05 73.96) (end 40.724744 73.96) (width 0.2) (layer "F.Cu") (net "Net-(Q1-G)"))
 (segment (start 49.04 73.96) (end 49 74) (width 0.2) (layer "F.Cu") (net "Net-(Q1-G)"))
 (segment (start 40.724744 73.96) (end 39.839744 73.075) (width 0.2) (layer "F.Cu") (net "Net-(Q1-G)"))
 (segment (start 39.839744 73.075) (end 36.095 73.075) (width 0.2) (layer "F.Cu") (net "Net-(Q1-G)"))
 (segment (start 49.05 73.96) (end 49.04 73.96) (width 0.2) (layer "F.Cu") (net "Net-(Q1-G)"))
 (segment (start 45.5 76.5) (end 47 76.5) (width 0.2) (layer "F.Cu") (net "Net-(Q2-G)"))
 (segment (start 34.025 77.025) (end 34 77) (width 0.2) (layer "F.Cu") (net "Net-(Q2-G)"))
 (segment (start 47 76.5) (end 49.05 76.5) (width 0.2) (layer "F.Cu") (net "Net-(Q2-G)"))
 (segment (start 34.025 78.695) (end 34.025 77.025) (width 0.2) (layer "F.Cu") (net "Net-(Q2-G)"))
 (via (at 47 76.5) (size 0.6) (drill 0.3) (layers "F.Cu" "B.Cu") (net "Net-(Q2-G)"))
 (via (at 34 77) (size 0.6) (drill 0.3) (layers "F.Cu" "B.Cu") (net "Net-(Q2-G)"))
 (segment (start 47 76.5) (end 34.5 76.5) (width 0.2) (layer "B.Cu") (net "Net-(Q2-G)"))
 (segment (start 34.5 76.5) (end 34 77) (width 0.2) (layer "B.Cu") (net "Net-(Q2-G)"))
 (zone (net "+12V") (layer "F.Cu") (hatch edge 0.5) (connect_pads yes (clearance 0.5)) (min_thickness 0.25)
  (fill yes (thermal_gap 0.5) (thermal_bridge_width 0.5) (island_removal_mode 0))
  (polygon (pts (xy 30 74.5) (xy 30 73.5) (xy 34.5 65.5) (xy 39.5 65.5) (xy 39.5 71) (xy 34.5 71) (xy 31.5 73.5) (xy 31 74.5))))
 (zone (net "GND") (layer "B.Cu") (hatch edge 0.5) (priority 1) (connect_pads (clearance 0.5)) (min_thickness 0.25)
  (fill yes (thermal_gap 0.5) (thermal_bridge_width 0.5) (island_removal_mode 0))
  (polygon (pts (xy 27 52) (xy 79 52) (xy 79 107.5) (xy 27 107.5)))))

